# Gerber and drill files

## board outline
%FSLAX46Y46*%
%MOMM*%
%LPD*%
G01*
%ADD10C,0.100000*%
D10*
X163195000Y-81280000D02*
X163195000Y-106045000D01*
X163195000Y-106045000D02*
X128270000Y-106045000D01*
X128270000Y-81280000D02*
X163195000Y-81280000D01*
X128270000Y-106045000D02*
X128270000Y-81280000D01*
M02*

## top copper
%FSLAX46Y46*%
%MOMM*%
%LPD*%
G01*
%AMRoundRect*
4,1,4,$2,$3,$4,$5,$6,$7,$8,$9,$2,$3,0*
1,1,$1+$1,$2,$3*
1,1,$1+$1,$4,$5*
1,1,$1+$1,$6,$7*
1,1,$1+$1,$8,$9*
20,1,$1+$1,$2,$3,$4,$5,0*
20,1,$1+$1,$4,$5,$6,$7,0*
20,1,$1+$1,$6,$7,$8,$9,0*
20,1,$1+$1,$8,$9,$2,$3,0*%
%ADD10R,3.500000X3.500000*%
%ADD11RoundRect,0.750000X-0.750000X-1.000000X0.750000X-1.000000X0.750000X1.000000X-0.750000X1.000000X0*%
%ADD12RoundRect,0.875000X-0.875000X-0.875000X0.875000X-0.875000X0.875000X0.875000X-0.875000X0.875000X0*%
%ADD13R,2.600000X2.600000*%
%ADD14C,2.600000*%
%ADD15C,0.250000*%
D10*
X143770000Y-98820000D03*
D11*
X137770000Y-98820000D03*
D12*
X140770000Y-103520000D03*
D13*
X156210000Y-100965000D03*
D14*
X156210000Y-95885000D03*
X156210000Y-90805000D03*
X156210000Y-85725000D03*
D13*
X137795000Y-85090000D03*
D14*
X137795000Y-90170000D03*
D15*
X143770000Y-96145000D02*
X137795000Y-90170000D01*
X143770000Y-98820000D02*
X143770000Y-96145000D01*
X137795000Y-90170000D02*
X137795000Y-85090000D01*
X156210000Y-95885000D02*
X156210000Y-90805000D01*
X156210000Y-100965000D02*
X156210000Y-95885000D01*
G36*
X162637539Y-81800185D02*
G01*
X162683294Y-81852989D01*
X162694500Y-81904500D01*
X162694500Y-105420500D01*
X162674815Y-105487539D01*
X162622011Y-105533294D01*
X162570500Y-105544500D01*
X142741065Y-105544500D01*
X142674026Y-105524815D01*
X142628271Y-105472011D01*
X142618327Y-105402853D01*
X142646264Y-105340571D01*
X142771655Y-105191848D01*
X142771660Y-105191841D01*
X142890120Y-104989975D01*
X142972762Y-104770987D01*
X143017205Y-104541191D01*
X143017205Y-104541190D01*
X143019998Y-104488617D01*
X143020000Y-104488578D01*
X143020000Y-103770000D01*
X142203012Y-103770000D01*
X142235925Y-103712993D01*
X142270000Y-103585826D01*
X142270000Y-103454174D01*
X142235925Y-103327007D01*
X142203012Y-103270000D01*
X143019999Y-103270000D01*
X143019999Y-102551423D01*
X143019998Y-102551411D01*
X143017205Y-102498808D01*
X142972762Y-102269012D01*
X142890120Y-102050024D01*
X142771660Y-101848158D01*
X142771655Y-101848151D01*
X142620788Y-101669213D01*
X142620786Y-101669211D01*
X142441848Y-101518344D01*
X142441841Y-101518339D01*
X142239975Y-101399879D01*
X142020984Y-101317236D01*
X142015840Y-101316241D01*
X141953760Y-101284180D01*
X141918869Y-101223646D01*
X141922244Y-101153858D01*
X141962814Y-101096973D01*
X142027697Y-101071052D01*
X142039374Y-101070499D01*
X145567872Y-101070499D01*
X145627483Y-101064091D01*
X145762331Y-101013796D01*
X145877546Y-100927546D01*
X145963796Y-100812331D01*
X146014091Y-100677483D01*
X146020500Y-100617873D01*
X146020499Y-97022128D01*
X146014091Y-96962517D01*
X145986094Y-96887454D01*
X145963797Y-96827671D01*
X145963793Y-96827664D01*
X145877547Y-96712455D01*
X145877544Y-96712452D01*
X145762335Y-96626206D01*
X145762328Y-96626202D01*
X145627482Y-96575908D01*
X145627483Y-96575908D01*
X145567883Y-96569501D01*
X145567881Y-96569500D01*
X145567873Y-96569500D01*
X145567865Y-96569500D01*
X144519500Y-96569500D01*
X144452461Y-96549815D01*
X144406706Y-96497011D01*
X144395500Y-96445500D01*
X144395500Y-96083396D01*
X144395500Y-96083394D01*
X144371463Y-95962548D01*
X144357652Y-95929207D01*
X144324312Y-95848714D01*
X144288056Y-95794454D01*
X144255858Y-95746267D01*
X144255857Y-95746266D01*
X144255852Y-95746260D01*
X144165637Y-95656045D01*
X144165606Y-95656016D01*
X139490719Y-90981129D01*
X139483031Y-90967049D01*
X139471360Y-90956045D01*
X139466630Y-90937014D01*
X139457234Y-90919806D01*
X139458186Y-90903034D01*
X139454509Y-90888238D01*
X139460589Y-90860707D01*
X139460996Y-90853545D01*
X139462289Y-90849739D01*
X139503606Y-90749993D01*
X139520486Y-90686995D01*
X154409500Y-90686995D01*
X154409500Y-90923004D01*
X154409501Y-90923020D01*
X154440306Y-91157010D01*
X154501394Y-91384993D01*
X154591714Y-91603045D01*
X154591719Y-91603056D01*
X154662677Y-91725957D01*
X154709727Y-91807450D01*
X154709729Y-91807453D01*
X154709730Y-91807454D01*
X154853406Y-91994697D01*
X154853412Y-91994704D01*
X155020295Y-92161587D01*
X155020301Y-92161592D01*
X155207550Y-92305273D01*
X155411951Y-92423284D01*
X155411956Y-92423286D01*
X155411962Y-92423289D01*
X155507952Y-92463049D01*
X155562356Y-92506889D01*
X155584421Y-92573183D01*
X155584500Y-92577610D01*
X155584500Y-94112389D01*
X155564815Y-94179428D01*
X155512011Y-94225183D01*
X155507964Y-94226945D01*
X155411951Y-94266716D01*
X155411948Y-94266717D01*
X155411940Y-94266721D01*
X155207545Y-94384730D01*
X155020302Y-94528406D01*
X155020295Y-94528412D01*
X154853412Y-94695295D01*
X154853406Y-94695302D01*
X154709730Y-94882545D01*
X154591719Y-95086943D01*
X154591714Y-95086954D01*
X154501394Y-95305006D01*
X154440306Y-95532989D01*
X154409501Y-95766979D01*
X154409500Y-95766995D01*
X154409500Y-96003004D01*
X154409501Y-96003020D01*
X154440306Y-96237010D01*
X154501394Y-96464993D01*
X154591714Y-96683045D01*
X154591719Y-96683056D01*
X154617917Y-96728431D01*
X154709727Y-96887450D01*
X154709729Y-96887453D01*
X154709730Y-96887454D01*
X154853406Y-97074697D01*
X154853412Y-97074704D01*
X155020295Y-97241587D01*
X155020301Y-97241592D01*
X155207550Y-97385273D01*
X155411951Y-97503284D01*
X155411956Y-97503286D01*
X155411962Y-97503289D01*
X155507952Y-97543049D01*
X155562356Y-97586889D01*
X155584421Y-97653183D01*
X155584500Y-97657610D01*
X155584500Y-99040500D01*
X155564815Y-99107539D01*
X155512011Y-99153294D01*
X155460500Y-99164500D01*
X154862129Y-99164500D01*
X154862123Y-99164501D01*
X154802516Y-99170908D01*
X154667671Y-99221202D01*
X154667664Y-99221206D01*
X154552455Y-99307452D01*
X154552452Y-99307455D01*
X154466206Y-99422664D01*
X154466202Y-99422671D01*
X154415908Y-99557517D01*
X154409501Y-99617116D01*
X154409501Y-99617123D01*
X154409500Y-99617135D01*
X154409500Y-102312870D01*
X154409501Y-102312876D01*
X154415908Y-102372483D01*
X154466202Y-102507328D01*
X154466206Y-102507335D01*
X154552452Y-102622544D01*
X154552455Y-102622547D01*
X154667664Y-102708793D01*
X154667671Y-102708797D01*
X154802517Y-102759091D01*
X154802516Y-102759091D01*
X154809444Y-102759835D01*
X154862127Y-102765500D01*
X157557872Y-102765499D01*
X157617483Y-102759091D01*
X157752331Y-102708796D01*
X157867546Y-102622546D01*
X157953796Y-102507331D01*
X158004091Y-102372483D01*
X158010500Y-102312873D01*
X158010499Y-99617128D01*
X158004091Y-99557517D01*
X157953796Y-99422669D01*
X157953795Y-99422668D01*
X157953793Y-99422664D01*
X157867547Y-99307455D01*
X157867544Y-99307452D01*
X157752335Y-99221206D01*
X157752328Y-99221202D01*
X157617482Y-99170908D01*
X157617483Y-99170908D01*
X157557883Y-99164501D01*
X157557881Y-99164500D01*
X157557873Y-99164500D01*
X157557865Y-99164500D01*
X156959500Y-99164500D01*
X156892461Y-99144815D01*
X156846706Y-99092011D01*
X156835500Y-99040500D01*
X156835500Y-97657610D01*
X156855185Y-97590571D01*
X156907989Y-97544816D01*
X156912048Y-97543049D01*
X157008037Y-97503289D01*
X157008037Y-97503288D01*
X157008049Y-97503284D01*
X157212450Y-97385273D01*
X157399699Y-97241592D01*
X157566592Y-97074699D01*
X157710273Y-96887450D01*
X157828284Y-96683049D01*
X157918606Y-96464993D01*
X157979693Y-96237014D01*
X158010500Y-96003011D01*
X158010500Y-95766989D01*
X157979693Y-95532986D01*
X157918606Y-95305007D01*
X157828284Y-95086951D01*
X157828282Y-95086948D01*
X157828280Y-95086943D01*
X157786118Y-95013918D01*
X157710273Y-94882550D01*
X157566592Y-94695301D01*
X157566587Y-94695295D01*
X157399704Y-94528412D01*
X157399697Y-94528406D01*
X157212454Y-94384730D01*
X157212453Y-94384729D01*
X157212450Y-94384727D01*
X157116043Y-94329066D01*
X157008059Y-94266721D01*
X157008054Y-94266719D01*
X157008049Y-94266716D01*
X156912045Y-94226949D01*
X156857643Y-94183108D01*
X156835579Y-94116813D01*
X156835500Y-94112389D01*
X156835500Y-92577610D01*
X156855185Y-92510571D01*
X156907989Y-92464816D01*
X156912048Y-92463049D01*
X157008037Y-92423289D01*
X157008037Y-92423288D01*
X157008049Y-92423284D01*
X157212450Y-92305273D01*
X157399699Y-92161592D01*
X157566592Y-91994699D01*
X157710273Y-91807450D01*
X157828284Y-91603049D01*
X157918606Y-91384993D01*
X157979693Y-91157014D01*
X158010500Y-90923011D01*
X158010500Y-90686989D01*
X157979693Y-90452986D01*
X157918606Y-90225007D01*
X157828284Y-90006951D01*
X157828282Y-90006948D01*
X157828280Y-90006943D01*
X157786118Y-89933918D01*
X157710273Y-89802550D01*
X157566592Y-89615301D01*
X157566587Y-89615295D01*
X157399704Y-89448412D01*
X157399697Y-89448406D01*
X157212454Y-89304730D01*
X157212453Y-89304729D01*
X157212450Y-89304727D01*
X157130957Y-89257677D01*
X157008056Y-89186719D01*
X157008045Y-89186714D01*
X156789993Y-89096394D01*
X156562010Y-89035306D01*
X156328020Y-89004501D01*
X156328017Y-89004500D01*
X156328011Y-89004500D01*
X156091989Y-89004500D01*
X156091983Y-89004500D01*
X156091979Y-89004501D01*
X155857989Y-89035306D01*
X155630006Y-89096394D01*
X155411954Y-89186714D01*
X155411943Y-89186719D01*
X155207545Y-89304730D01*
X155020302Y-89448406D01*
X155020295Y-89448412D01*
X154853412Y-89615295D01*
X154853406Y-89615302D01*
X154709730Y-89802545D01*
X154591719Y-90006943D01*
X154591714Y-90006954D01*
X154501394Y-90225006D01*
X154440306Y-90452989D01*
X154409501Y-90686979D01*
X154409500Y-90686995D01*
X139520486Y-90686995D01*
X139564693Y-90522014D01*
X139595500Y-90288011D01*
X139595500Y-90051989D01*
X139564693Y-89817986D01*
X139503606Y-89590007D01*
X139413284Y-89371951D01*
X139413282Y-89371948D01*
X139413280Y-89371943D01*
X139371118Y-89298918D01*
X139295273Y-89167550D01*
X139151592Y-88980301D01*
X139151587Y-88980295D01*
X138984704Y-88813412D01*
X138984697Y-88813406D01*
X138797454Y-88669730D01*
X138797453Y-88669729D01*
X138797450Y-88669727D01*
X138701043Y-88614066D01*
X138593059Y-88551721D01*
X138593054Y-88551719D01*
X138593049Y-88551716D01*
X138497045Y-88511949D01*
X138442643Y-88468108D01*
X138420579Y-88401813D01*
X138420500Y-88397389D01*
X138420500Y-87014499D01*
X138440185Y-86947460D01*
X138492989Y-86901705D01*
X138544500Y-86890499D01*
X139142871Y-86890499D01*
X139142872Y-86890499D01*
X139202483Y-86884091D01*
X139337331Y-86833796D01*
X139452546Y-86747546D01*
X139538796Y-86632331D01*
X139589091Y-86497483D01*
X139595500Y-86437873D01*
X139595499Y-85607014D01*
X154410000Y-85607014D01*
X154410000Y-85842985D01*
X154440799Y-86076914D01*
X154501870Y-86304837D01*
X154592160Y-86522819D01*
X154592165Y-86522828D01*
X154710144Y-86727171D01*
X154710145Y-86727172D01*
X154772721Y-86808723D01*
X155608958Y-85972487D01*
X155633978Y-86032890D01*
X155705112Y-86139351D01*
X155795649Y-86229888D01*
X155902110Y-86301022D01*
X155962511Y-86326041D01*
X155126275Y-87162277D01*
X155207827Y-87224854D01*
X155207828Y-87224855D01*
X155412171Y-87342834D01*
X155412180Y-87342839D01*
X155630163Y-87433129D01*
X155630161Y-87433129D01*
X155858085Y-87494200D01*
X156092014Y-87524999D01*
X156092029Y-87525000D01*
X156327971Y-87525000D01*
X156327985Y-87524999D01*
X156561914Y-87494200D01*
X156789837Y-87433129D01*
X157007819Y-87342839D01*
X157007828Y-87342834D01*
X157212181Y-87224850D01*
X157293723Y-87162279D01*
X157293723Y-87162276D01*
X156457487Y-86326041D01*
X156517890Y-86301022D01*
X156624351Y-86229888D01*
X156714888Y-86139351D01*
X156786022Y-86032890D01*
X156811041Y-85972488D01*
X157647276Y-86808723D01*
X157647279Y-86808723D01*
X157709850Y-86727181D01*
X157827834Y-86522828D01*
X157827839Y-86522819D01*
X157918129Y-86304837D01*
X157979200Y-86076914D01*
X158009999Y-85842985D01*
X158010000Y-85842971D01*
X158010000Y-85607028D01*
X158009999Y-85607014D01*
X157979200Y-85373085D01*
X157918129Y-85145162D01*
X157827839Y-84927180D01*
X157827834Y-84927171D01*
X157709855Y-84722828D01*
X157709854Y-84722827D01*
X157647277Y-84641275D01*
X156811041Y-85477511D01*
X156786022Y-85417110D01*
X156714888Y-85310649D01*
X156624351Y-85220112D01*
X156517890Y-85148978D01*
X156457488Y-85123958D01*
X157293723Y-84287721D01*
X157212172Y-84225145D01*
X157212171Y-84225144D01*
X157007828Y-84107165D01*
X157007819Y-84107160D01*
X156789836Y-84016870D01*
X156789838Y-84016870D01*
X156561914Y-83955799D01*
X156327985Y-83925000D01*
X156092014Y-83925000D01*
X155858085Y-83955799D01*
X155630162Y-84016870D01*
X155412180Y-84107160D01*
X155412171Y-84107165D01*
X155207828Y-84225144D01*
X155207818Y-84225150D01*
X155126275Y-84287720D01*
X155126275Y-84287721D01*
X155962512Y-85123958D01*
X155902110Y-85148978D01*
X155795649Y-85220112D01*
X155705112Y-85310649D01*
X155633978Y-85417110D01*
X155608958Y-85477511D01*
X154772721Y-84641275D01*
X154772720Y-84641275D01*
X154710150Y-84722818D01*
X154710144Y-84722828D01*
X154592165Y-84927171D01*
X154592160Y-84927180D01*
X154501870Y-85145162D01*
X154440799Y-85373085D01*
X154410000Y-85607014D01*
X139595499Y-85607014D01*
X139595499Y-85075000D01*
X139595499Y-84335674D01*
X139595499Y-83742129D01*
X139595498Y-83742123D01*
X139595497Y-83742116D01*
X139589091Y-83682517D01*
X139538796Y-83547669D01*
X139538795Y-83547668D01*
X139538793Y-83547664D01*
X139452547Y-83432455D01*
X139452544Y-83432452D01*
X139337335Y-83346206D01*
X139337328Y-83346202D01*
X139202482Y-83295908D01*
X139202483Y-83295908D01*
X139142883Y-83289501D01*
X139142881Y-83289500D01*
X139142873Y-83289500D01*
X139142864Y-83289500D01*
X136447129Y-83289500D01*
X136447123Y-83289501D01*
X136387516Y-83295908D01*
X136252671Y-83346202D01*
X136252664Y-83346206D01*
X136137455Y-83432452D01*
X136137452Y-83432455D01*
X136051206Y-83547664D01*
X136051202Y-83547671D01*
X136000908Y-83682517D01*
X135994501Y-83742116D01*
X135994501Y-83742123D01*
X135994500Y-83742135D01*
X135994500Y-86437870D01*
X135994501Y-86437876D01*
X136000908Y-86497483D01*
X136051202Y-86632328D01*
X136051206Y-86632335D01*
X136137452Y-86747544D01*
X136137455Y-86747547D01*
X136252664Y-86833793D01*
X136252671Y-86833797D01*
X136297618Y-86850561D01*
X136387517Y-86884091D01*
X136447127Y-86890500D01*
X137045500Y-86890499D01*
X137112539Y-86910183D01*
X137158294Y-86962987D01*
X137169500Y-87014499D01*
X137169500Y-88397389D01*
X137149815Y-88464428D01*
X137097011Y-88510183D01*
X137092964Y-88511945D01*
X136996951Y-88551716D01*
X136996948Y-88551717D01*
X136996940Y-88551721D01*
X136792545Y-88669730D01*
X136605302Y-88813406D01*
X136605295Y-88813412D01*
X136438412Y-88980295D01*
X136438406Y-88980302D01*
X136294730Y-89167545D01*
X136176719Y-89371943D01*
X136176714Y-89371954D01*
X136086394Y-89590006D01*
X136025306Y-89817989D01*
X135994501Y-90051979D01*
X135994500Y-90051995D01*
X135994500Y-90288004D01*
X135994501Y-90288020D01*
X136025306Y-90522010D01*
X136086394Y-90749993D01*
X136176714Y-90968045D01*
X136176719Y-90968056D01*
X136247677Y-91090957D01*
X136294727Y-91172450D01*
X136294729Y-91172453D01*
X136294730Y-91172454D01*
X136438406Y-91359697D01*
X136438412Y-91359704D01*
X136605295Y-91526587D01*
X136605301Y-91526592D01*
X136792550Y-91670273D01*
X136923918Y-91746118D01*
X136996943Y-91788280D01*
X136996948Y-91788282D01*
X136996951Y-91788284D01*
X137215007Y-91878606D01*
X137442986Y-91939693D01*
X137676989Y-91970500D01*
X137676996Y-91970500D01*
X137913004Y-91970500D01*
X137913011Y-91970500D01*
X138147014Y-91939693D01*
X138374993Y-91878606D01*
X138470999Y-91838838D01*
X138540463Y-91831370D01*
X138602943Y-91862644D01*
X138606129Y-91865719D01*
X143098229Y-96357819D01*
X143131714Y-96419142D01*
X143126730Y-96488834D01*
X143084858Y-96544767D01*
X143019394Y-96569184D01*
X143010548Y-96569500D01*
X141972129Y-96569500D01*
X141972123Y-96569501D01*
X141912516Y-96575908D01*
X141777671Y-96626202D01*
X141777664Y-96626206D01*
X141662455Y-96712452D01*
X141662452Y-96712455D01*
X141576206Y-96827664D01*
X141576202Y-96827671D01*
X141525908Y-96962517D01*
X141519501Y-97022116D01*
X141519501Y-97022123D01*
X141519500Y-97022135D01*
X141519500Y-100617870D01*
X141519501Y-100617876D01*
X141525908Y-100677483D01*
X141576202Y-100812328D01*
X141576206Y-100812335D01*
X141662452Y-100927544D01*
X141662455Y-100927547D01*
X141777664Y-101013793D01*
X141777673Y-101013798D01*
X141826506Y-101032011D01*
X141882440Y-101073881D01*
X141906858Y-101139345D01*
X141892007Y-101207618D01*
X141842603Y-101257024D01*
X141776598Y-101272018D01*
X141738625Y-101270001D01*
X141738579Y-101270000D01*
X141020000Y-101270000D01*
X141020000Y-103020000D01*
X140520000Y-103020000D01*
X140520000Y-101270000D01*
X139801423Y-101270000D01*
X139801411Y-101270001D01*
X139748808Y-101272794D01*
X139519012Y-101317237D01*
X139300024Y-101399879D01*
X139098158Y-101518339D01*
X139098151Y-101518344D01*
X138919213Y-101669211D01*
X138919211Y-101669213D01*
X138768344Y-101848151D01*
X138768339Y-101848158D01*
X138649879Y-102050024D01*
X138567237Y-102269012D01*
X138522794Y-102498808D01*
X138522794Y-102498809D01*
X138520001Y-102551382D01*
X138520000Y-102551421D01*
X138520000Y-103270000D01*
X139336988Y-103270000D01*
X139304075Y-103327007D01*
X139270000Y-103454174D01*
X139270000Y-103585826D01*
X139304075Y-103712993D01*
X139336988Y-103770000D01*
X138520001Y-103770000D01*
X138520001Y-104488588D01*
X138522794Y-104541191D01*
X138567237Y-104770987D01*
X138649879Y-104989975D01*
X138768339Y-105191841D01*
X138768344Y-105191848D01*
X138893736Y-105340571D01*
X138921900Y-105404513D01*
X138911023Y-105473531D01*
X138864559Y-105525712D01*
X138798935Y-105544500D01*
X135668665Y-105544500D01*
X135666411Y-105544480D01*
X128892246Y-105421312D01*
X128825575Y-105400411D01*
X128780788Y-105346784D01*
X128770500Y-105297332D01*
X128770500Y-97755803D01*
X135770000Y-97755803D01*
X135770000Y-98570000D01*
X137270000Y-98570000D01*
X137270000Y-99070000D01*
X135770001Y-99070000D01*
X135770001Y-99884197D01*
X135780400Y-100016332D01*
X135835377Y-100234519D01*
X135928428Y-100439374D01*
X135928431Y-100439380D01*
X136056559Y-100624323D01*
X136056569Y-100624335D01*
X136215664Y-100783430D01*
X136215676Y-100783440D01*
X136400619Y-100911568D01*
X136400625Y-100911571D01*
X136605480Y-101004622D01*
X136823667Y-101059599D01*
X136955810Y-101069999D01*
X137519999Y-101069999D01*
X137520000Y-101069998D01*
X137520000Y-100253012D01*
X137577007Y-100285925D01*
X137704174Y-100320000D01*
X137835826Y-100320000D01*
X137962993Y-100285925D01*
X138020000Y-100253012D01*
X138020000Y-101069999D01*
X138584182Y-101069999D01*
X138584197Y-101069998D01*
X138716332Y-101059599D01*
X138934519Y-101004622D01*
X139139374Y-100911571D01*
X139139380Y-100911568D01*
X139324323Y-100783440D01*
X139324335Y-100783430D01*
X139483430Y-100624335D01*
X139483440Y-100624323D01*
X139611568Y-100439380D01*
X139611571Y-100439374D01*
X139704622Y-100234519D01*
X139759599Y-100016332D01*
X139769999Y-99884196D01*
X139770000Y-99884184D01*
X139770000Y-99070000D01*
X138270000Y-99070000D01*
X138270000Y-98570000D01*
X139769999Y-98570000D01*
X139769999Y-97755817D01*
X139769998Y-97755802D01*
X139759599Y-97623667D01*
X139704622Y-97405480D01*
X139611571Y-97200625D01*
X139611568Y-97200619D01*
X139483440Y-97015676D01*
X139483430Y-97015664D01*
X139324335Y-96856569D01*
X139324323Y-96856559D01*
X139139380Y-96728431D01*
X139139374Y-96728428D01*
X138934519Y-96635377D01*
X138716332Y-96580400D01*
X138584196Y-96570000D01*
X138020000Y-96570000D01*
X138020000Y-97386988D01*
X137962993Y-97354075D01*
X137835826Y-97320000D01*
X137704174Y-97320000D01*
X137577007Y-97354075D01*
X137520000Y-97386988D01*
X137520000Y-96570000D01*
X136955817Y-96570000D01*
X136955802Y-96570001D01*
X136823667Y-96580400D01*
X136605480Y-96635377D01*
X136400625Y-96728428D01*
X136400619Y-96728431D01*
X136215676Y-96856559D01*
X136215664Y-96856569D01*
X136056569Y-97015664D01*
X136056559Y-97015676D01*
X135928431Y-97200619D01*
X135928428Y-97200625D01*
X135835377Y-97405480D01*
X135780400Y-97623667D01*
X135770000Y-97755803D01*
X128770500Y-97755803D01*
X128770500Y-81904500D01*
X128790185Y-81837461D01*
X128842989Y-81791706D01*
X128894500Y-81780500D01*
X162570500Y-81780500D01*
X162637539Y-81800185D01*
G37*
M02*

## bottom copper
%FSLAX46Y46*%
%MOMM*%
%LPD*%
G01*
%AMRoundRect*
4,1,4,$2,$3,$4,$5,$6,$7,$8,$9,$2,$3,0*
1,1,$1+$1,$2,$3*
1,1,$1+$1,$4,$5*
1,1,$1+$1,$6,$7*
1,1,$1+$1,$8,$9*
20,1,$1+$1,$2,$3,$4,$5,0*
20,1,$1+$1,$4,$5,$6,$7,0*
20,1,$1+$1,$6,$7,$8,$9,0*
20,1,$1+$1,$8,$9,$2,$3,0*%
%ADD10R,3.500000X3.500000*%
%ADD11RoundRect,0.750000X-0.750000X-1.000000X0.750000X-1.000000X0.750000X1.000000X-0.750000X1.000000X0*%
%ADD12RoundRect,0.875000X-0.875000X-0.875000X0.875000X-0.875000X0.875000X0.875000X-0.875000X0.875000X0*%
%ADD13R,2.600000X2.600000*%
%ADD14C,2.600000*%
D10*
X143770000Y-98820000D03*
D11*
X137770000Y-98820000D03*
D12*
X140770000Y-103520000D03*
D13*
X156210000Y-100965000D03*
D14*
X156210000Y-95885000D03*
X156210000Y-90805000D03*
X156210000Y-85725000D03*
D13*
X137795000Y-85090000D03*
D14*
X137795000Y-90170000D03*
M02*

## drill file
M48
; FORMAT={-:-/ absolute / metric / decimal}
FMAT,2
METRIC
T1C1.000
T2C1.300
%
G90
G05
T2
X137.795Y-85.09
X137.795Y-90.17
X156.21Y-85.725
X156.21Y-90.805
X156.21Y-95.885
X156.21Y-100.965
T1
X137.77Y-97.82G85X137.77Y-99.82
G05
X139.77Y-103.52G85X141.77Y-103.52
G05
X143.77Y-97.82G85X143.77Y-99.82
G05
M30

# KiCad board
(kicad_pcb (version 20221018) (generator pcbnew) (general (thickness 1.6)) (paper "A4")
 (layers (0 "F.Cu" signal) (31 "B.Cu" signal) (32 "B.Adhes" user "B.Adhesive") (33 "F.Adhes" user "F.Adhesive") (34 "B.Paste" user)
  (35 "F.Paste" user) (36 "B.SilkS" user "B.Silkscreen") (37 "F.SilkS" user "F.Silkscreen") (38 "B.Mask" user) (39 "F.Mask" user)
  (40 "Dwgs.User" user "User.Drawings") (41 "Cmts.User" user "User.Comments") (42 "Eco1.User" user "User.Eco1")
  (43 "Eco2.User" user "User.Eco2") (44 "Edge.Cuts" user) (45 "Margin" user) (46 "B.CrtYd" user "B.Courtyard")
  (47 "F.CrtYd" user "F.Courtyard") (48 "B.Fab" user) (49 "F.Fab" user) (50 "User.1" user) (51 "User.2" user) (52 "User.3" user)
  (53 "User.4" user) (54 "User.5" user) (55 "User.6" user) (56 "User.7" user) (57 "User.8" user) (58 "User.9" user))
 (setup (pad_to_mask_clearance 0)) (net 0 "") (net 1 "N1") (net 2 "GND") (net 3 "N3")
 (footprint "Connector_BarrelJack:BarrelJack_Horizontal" (layer "F.Cu") (at 143.77 98.82)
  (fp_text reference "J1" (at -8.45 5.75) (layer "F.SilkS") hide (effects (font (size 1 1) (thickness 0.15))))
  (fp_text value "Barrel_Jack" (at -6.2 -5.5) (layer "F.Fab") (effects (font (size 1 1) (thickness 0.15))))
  (pad "1" thru_hole rect (at 0 0) (size 3.5 3.5) (drill oval 1 3) (layers "*.Cu" "*.Mask") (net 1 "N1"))
  (pad "2" thru_hole roundrect (at -6 0) (size 3 3.5) (drill oval 1 3) (layers "*.Cu" "*.Mask") (roundrect_rratio 0.25) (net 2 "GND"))
  (pad "3" thru_hole roundrect (at -3 4.7) (size 3.5 3.5) (drill oval 3 1) (layers "*.Cu" "*.Mask") (roundrect_rratio 0.25) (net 2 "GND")))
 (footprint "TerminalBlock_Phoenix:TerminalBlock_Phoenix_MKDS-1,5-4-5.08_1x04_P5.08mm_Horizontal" (layer "F.Cu") (at 156.21 100.965 90)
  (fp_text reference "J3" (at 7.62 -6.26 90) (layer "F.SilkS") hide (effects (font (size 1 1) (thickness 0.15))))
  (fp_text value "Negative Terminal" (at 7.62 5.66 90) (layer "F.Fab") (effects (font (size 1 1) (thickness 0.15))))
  (pad "1" thru_hole rect (at 0 0 90) (size 2.6 2.6) (drill 1.3) (layers "*.Cu" "*.Mask") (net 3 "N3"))
  (pad "2" thru_hole circle (at 5.08 0 90) (size 2.6 2.6) (drill 1.3) (layers "*.Cu" "*.Mask") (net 3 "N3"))
  (pad "3" thru_hole circle (at 10.16 0 90) (size 2.6 2.6) (drill 1.3) (layers "*.Cu" "*.Mask") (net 3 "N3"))
  (pad "4" thru_hole circle (at 15.24 0 90) (size 2.6 2.6) (drill 1.3) (layers "*.Cu" "*.Mask") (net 2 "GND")))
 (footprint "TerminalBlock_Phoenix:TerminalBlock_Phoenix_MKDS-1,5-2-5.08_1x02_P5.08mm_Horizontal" (layer "F.Cu") (at 137.795 85.09 -90)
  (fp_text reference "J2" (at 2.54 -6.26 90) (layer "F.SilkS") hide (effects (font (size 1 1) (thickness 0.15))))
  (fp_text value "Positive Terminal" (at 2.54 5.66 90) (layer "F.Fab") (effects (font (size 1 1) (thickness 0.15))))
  (pad "1" thru_hole rect (at 0 0 270) (size 2.6 2.6) (drill 1.3) (layers "*.Cu" "*.Mask") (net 1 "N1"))
  (pad "2" thru_hole circle (at 5.08 0 270) (size 2.6 2.6) (drill 1.3) (layers "*.Cu" "*.Mask") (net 1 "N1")))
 (gr_line (start 163.195 81.28) (end 163.195 106.045) (stroke (width 0.1) (type default)) (layer "Edge.Cuts"))
 (gr_line (start 163.195 106.045) (end 128.27 106.045) (stroke (width 0.1) (type default)) (layer "Edge.Cuts"))
 (gr_line (start 128.27 81.28) (end 163.195 81.28) (stroke (width 0.1) (type default)) (layer "Edge.Cuts"))
 (gr_line (start 128.27 106.045) (end 128.27 81.28) (stroke (width 0.1) (type default)) (layer "Edge.Cuts"))
 (segment (start 143.77 96.145) (end 137.795 90.17) (width 0.25) (layer "F.Cu") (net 1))
 (segment (start 143.77 98.82) (end 143.77 96.145) (width 0.25) (layer "F.Cu") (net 1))
 (segment (start 137.795 90.17) (end 137.795 85.09) (width 0.25) (layer "F.Cu") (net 1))
 (segment (start 156.21 95.885) (end 156.21 90.805) (width 0.25) (layer "F.Cu") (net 3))
 (segment (start 156.21 100.965) (end 156.21 95.885) (width 0.25) (layer "F.Cu") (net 3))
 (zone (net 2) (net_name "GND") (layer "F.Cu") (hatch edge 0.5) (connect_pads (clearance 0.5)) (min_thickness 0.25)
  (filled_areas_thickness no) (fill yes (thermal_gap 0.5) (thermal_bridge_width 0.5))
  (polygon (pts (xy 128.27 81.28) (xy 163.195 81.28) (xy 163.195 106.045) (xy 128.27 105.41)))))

